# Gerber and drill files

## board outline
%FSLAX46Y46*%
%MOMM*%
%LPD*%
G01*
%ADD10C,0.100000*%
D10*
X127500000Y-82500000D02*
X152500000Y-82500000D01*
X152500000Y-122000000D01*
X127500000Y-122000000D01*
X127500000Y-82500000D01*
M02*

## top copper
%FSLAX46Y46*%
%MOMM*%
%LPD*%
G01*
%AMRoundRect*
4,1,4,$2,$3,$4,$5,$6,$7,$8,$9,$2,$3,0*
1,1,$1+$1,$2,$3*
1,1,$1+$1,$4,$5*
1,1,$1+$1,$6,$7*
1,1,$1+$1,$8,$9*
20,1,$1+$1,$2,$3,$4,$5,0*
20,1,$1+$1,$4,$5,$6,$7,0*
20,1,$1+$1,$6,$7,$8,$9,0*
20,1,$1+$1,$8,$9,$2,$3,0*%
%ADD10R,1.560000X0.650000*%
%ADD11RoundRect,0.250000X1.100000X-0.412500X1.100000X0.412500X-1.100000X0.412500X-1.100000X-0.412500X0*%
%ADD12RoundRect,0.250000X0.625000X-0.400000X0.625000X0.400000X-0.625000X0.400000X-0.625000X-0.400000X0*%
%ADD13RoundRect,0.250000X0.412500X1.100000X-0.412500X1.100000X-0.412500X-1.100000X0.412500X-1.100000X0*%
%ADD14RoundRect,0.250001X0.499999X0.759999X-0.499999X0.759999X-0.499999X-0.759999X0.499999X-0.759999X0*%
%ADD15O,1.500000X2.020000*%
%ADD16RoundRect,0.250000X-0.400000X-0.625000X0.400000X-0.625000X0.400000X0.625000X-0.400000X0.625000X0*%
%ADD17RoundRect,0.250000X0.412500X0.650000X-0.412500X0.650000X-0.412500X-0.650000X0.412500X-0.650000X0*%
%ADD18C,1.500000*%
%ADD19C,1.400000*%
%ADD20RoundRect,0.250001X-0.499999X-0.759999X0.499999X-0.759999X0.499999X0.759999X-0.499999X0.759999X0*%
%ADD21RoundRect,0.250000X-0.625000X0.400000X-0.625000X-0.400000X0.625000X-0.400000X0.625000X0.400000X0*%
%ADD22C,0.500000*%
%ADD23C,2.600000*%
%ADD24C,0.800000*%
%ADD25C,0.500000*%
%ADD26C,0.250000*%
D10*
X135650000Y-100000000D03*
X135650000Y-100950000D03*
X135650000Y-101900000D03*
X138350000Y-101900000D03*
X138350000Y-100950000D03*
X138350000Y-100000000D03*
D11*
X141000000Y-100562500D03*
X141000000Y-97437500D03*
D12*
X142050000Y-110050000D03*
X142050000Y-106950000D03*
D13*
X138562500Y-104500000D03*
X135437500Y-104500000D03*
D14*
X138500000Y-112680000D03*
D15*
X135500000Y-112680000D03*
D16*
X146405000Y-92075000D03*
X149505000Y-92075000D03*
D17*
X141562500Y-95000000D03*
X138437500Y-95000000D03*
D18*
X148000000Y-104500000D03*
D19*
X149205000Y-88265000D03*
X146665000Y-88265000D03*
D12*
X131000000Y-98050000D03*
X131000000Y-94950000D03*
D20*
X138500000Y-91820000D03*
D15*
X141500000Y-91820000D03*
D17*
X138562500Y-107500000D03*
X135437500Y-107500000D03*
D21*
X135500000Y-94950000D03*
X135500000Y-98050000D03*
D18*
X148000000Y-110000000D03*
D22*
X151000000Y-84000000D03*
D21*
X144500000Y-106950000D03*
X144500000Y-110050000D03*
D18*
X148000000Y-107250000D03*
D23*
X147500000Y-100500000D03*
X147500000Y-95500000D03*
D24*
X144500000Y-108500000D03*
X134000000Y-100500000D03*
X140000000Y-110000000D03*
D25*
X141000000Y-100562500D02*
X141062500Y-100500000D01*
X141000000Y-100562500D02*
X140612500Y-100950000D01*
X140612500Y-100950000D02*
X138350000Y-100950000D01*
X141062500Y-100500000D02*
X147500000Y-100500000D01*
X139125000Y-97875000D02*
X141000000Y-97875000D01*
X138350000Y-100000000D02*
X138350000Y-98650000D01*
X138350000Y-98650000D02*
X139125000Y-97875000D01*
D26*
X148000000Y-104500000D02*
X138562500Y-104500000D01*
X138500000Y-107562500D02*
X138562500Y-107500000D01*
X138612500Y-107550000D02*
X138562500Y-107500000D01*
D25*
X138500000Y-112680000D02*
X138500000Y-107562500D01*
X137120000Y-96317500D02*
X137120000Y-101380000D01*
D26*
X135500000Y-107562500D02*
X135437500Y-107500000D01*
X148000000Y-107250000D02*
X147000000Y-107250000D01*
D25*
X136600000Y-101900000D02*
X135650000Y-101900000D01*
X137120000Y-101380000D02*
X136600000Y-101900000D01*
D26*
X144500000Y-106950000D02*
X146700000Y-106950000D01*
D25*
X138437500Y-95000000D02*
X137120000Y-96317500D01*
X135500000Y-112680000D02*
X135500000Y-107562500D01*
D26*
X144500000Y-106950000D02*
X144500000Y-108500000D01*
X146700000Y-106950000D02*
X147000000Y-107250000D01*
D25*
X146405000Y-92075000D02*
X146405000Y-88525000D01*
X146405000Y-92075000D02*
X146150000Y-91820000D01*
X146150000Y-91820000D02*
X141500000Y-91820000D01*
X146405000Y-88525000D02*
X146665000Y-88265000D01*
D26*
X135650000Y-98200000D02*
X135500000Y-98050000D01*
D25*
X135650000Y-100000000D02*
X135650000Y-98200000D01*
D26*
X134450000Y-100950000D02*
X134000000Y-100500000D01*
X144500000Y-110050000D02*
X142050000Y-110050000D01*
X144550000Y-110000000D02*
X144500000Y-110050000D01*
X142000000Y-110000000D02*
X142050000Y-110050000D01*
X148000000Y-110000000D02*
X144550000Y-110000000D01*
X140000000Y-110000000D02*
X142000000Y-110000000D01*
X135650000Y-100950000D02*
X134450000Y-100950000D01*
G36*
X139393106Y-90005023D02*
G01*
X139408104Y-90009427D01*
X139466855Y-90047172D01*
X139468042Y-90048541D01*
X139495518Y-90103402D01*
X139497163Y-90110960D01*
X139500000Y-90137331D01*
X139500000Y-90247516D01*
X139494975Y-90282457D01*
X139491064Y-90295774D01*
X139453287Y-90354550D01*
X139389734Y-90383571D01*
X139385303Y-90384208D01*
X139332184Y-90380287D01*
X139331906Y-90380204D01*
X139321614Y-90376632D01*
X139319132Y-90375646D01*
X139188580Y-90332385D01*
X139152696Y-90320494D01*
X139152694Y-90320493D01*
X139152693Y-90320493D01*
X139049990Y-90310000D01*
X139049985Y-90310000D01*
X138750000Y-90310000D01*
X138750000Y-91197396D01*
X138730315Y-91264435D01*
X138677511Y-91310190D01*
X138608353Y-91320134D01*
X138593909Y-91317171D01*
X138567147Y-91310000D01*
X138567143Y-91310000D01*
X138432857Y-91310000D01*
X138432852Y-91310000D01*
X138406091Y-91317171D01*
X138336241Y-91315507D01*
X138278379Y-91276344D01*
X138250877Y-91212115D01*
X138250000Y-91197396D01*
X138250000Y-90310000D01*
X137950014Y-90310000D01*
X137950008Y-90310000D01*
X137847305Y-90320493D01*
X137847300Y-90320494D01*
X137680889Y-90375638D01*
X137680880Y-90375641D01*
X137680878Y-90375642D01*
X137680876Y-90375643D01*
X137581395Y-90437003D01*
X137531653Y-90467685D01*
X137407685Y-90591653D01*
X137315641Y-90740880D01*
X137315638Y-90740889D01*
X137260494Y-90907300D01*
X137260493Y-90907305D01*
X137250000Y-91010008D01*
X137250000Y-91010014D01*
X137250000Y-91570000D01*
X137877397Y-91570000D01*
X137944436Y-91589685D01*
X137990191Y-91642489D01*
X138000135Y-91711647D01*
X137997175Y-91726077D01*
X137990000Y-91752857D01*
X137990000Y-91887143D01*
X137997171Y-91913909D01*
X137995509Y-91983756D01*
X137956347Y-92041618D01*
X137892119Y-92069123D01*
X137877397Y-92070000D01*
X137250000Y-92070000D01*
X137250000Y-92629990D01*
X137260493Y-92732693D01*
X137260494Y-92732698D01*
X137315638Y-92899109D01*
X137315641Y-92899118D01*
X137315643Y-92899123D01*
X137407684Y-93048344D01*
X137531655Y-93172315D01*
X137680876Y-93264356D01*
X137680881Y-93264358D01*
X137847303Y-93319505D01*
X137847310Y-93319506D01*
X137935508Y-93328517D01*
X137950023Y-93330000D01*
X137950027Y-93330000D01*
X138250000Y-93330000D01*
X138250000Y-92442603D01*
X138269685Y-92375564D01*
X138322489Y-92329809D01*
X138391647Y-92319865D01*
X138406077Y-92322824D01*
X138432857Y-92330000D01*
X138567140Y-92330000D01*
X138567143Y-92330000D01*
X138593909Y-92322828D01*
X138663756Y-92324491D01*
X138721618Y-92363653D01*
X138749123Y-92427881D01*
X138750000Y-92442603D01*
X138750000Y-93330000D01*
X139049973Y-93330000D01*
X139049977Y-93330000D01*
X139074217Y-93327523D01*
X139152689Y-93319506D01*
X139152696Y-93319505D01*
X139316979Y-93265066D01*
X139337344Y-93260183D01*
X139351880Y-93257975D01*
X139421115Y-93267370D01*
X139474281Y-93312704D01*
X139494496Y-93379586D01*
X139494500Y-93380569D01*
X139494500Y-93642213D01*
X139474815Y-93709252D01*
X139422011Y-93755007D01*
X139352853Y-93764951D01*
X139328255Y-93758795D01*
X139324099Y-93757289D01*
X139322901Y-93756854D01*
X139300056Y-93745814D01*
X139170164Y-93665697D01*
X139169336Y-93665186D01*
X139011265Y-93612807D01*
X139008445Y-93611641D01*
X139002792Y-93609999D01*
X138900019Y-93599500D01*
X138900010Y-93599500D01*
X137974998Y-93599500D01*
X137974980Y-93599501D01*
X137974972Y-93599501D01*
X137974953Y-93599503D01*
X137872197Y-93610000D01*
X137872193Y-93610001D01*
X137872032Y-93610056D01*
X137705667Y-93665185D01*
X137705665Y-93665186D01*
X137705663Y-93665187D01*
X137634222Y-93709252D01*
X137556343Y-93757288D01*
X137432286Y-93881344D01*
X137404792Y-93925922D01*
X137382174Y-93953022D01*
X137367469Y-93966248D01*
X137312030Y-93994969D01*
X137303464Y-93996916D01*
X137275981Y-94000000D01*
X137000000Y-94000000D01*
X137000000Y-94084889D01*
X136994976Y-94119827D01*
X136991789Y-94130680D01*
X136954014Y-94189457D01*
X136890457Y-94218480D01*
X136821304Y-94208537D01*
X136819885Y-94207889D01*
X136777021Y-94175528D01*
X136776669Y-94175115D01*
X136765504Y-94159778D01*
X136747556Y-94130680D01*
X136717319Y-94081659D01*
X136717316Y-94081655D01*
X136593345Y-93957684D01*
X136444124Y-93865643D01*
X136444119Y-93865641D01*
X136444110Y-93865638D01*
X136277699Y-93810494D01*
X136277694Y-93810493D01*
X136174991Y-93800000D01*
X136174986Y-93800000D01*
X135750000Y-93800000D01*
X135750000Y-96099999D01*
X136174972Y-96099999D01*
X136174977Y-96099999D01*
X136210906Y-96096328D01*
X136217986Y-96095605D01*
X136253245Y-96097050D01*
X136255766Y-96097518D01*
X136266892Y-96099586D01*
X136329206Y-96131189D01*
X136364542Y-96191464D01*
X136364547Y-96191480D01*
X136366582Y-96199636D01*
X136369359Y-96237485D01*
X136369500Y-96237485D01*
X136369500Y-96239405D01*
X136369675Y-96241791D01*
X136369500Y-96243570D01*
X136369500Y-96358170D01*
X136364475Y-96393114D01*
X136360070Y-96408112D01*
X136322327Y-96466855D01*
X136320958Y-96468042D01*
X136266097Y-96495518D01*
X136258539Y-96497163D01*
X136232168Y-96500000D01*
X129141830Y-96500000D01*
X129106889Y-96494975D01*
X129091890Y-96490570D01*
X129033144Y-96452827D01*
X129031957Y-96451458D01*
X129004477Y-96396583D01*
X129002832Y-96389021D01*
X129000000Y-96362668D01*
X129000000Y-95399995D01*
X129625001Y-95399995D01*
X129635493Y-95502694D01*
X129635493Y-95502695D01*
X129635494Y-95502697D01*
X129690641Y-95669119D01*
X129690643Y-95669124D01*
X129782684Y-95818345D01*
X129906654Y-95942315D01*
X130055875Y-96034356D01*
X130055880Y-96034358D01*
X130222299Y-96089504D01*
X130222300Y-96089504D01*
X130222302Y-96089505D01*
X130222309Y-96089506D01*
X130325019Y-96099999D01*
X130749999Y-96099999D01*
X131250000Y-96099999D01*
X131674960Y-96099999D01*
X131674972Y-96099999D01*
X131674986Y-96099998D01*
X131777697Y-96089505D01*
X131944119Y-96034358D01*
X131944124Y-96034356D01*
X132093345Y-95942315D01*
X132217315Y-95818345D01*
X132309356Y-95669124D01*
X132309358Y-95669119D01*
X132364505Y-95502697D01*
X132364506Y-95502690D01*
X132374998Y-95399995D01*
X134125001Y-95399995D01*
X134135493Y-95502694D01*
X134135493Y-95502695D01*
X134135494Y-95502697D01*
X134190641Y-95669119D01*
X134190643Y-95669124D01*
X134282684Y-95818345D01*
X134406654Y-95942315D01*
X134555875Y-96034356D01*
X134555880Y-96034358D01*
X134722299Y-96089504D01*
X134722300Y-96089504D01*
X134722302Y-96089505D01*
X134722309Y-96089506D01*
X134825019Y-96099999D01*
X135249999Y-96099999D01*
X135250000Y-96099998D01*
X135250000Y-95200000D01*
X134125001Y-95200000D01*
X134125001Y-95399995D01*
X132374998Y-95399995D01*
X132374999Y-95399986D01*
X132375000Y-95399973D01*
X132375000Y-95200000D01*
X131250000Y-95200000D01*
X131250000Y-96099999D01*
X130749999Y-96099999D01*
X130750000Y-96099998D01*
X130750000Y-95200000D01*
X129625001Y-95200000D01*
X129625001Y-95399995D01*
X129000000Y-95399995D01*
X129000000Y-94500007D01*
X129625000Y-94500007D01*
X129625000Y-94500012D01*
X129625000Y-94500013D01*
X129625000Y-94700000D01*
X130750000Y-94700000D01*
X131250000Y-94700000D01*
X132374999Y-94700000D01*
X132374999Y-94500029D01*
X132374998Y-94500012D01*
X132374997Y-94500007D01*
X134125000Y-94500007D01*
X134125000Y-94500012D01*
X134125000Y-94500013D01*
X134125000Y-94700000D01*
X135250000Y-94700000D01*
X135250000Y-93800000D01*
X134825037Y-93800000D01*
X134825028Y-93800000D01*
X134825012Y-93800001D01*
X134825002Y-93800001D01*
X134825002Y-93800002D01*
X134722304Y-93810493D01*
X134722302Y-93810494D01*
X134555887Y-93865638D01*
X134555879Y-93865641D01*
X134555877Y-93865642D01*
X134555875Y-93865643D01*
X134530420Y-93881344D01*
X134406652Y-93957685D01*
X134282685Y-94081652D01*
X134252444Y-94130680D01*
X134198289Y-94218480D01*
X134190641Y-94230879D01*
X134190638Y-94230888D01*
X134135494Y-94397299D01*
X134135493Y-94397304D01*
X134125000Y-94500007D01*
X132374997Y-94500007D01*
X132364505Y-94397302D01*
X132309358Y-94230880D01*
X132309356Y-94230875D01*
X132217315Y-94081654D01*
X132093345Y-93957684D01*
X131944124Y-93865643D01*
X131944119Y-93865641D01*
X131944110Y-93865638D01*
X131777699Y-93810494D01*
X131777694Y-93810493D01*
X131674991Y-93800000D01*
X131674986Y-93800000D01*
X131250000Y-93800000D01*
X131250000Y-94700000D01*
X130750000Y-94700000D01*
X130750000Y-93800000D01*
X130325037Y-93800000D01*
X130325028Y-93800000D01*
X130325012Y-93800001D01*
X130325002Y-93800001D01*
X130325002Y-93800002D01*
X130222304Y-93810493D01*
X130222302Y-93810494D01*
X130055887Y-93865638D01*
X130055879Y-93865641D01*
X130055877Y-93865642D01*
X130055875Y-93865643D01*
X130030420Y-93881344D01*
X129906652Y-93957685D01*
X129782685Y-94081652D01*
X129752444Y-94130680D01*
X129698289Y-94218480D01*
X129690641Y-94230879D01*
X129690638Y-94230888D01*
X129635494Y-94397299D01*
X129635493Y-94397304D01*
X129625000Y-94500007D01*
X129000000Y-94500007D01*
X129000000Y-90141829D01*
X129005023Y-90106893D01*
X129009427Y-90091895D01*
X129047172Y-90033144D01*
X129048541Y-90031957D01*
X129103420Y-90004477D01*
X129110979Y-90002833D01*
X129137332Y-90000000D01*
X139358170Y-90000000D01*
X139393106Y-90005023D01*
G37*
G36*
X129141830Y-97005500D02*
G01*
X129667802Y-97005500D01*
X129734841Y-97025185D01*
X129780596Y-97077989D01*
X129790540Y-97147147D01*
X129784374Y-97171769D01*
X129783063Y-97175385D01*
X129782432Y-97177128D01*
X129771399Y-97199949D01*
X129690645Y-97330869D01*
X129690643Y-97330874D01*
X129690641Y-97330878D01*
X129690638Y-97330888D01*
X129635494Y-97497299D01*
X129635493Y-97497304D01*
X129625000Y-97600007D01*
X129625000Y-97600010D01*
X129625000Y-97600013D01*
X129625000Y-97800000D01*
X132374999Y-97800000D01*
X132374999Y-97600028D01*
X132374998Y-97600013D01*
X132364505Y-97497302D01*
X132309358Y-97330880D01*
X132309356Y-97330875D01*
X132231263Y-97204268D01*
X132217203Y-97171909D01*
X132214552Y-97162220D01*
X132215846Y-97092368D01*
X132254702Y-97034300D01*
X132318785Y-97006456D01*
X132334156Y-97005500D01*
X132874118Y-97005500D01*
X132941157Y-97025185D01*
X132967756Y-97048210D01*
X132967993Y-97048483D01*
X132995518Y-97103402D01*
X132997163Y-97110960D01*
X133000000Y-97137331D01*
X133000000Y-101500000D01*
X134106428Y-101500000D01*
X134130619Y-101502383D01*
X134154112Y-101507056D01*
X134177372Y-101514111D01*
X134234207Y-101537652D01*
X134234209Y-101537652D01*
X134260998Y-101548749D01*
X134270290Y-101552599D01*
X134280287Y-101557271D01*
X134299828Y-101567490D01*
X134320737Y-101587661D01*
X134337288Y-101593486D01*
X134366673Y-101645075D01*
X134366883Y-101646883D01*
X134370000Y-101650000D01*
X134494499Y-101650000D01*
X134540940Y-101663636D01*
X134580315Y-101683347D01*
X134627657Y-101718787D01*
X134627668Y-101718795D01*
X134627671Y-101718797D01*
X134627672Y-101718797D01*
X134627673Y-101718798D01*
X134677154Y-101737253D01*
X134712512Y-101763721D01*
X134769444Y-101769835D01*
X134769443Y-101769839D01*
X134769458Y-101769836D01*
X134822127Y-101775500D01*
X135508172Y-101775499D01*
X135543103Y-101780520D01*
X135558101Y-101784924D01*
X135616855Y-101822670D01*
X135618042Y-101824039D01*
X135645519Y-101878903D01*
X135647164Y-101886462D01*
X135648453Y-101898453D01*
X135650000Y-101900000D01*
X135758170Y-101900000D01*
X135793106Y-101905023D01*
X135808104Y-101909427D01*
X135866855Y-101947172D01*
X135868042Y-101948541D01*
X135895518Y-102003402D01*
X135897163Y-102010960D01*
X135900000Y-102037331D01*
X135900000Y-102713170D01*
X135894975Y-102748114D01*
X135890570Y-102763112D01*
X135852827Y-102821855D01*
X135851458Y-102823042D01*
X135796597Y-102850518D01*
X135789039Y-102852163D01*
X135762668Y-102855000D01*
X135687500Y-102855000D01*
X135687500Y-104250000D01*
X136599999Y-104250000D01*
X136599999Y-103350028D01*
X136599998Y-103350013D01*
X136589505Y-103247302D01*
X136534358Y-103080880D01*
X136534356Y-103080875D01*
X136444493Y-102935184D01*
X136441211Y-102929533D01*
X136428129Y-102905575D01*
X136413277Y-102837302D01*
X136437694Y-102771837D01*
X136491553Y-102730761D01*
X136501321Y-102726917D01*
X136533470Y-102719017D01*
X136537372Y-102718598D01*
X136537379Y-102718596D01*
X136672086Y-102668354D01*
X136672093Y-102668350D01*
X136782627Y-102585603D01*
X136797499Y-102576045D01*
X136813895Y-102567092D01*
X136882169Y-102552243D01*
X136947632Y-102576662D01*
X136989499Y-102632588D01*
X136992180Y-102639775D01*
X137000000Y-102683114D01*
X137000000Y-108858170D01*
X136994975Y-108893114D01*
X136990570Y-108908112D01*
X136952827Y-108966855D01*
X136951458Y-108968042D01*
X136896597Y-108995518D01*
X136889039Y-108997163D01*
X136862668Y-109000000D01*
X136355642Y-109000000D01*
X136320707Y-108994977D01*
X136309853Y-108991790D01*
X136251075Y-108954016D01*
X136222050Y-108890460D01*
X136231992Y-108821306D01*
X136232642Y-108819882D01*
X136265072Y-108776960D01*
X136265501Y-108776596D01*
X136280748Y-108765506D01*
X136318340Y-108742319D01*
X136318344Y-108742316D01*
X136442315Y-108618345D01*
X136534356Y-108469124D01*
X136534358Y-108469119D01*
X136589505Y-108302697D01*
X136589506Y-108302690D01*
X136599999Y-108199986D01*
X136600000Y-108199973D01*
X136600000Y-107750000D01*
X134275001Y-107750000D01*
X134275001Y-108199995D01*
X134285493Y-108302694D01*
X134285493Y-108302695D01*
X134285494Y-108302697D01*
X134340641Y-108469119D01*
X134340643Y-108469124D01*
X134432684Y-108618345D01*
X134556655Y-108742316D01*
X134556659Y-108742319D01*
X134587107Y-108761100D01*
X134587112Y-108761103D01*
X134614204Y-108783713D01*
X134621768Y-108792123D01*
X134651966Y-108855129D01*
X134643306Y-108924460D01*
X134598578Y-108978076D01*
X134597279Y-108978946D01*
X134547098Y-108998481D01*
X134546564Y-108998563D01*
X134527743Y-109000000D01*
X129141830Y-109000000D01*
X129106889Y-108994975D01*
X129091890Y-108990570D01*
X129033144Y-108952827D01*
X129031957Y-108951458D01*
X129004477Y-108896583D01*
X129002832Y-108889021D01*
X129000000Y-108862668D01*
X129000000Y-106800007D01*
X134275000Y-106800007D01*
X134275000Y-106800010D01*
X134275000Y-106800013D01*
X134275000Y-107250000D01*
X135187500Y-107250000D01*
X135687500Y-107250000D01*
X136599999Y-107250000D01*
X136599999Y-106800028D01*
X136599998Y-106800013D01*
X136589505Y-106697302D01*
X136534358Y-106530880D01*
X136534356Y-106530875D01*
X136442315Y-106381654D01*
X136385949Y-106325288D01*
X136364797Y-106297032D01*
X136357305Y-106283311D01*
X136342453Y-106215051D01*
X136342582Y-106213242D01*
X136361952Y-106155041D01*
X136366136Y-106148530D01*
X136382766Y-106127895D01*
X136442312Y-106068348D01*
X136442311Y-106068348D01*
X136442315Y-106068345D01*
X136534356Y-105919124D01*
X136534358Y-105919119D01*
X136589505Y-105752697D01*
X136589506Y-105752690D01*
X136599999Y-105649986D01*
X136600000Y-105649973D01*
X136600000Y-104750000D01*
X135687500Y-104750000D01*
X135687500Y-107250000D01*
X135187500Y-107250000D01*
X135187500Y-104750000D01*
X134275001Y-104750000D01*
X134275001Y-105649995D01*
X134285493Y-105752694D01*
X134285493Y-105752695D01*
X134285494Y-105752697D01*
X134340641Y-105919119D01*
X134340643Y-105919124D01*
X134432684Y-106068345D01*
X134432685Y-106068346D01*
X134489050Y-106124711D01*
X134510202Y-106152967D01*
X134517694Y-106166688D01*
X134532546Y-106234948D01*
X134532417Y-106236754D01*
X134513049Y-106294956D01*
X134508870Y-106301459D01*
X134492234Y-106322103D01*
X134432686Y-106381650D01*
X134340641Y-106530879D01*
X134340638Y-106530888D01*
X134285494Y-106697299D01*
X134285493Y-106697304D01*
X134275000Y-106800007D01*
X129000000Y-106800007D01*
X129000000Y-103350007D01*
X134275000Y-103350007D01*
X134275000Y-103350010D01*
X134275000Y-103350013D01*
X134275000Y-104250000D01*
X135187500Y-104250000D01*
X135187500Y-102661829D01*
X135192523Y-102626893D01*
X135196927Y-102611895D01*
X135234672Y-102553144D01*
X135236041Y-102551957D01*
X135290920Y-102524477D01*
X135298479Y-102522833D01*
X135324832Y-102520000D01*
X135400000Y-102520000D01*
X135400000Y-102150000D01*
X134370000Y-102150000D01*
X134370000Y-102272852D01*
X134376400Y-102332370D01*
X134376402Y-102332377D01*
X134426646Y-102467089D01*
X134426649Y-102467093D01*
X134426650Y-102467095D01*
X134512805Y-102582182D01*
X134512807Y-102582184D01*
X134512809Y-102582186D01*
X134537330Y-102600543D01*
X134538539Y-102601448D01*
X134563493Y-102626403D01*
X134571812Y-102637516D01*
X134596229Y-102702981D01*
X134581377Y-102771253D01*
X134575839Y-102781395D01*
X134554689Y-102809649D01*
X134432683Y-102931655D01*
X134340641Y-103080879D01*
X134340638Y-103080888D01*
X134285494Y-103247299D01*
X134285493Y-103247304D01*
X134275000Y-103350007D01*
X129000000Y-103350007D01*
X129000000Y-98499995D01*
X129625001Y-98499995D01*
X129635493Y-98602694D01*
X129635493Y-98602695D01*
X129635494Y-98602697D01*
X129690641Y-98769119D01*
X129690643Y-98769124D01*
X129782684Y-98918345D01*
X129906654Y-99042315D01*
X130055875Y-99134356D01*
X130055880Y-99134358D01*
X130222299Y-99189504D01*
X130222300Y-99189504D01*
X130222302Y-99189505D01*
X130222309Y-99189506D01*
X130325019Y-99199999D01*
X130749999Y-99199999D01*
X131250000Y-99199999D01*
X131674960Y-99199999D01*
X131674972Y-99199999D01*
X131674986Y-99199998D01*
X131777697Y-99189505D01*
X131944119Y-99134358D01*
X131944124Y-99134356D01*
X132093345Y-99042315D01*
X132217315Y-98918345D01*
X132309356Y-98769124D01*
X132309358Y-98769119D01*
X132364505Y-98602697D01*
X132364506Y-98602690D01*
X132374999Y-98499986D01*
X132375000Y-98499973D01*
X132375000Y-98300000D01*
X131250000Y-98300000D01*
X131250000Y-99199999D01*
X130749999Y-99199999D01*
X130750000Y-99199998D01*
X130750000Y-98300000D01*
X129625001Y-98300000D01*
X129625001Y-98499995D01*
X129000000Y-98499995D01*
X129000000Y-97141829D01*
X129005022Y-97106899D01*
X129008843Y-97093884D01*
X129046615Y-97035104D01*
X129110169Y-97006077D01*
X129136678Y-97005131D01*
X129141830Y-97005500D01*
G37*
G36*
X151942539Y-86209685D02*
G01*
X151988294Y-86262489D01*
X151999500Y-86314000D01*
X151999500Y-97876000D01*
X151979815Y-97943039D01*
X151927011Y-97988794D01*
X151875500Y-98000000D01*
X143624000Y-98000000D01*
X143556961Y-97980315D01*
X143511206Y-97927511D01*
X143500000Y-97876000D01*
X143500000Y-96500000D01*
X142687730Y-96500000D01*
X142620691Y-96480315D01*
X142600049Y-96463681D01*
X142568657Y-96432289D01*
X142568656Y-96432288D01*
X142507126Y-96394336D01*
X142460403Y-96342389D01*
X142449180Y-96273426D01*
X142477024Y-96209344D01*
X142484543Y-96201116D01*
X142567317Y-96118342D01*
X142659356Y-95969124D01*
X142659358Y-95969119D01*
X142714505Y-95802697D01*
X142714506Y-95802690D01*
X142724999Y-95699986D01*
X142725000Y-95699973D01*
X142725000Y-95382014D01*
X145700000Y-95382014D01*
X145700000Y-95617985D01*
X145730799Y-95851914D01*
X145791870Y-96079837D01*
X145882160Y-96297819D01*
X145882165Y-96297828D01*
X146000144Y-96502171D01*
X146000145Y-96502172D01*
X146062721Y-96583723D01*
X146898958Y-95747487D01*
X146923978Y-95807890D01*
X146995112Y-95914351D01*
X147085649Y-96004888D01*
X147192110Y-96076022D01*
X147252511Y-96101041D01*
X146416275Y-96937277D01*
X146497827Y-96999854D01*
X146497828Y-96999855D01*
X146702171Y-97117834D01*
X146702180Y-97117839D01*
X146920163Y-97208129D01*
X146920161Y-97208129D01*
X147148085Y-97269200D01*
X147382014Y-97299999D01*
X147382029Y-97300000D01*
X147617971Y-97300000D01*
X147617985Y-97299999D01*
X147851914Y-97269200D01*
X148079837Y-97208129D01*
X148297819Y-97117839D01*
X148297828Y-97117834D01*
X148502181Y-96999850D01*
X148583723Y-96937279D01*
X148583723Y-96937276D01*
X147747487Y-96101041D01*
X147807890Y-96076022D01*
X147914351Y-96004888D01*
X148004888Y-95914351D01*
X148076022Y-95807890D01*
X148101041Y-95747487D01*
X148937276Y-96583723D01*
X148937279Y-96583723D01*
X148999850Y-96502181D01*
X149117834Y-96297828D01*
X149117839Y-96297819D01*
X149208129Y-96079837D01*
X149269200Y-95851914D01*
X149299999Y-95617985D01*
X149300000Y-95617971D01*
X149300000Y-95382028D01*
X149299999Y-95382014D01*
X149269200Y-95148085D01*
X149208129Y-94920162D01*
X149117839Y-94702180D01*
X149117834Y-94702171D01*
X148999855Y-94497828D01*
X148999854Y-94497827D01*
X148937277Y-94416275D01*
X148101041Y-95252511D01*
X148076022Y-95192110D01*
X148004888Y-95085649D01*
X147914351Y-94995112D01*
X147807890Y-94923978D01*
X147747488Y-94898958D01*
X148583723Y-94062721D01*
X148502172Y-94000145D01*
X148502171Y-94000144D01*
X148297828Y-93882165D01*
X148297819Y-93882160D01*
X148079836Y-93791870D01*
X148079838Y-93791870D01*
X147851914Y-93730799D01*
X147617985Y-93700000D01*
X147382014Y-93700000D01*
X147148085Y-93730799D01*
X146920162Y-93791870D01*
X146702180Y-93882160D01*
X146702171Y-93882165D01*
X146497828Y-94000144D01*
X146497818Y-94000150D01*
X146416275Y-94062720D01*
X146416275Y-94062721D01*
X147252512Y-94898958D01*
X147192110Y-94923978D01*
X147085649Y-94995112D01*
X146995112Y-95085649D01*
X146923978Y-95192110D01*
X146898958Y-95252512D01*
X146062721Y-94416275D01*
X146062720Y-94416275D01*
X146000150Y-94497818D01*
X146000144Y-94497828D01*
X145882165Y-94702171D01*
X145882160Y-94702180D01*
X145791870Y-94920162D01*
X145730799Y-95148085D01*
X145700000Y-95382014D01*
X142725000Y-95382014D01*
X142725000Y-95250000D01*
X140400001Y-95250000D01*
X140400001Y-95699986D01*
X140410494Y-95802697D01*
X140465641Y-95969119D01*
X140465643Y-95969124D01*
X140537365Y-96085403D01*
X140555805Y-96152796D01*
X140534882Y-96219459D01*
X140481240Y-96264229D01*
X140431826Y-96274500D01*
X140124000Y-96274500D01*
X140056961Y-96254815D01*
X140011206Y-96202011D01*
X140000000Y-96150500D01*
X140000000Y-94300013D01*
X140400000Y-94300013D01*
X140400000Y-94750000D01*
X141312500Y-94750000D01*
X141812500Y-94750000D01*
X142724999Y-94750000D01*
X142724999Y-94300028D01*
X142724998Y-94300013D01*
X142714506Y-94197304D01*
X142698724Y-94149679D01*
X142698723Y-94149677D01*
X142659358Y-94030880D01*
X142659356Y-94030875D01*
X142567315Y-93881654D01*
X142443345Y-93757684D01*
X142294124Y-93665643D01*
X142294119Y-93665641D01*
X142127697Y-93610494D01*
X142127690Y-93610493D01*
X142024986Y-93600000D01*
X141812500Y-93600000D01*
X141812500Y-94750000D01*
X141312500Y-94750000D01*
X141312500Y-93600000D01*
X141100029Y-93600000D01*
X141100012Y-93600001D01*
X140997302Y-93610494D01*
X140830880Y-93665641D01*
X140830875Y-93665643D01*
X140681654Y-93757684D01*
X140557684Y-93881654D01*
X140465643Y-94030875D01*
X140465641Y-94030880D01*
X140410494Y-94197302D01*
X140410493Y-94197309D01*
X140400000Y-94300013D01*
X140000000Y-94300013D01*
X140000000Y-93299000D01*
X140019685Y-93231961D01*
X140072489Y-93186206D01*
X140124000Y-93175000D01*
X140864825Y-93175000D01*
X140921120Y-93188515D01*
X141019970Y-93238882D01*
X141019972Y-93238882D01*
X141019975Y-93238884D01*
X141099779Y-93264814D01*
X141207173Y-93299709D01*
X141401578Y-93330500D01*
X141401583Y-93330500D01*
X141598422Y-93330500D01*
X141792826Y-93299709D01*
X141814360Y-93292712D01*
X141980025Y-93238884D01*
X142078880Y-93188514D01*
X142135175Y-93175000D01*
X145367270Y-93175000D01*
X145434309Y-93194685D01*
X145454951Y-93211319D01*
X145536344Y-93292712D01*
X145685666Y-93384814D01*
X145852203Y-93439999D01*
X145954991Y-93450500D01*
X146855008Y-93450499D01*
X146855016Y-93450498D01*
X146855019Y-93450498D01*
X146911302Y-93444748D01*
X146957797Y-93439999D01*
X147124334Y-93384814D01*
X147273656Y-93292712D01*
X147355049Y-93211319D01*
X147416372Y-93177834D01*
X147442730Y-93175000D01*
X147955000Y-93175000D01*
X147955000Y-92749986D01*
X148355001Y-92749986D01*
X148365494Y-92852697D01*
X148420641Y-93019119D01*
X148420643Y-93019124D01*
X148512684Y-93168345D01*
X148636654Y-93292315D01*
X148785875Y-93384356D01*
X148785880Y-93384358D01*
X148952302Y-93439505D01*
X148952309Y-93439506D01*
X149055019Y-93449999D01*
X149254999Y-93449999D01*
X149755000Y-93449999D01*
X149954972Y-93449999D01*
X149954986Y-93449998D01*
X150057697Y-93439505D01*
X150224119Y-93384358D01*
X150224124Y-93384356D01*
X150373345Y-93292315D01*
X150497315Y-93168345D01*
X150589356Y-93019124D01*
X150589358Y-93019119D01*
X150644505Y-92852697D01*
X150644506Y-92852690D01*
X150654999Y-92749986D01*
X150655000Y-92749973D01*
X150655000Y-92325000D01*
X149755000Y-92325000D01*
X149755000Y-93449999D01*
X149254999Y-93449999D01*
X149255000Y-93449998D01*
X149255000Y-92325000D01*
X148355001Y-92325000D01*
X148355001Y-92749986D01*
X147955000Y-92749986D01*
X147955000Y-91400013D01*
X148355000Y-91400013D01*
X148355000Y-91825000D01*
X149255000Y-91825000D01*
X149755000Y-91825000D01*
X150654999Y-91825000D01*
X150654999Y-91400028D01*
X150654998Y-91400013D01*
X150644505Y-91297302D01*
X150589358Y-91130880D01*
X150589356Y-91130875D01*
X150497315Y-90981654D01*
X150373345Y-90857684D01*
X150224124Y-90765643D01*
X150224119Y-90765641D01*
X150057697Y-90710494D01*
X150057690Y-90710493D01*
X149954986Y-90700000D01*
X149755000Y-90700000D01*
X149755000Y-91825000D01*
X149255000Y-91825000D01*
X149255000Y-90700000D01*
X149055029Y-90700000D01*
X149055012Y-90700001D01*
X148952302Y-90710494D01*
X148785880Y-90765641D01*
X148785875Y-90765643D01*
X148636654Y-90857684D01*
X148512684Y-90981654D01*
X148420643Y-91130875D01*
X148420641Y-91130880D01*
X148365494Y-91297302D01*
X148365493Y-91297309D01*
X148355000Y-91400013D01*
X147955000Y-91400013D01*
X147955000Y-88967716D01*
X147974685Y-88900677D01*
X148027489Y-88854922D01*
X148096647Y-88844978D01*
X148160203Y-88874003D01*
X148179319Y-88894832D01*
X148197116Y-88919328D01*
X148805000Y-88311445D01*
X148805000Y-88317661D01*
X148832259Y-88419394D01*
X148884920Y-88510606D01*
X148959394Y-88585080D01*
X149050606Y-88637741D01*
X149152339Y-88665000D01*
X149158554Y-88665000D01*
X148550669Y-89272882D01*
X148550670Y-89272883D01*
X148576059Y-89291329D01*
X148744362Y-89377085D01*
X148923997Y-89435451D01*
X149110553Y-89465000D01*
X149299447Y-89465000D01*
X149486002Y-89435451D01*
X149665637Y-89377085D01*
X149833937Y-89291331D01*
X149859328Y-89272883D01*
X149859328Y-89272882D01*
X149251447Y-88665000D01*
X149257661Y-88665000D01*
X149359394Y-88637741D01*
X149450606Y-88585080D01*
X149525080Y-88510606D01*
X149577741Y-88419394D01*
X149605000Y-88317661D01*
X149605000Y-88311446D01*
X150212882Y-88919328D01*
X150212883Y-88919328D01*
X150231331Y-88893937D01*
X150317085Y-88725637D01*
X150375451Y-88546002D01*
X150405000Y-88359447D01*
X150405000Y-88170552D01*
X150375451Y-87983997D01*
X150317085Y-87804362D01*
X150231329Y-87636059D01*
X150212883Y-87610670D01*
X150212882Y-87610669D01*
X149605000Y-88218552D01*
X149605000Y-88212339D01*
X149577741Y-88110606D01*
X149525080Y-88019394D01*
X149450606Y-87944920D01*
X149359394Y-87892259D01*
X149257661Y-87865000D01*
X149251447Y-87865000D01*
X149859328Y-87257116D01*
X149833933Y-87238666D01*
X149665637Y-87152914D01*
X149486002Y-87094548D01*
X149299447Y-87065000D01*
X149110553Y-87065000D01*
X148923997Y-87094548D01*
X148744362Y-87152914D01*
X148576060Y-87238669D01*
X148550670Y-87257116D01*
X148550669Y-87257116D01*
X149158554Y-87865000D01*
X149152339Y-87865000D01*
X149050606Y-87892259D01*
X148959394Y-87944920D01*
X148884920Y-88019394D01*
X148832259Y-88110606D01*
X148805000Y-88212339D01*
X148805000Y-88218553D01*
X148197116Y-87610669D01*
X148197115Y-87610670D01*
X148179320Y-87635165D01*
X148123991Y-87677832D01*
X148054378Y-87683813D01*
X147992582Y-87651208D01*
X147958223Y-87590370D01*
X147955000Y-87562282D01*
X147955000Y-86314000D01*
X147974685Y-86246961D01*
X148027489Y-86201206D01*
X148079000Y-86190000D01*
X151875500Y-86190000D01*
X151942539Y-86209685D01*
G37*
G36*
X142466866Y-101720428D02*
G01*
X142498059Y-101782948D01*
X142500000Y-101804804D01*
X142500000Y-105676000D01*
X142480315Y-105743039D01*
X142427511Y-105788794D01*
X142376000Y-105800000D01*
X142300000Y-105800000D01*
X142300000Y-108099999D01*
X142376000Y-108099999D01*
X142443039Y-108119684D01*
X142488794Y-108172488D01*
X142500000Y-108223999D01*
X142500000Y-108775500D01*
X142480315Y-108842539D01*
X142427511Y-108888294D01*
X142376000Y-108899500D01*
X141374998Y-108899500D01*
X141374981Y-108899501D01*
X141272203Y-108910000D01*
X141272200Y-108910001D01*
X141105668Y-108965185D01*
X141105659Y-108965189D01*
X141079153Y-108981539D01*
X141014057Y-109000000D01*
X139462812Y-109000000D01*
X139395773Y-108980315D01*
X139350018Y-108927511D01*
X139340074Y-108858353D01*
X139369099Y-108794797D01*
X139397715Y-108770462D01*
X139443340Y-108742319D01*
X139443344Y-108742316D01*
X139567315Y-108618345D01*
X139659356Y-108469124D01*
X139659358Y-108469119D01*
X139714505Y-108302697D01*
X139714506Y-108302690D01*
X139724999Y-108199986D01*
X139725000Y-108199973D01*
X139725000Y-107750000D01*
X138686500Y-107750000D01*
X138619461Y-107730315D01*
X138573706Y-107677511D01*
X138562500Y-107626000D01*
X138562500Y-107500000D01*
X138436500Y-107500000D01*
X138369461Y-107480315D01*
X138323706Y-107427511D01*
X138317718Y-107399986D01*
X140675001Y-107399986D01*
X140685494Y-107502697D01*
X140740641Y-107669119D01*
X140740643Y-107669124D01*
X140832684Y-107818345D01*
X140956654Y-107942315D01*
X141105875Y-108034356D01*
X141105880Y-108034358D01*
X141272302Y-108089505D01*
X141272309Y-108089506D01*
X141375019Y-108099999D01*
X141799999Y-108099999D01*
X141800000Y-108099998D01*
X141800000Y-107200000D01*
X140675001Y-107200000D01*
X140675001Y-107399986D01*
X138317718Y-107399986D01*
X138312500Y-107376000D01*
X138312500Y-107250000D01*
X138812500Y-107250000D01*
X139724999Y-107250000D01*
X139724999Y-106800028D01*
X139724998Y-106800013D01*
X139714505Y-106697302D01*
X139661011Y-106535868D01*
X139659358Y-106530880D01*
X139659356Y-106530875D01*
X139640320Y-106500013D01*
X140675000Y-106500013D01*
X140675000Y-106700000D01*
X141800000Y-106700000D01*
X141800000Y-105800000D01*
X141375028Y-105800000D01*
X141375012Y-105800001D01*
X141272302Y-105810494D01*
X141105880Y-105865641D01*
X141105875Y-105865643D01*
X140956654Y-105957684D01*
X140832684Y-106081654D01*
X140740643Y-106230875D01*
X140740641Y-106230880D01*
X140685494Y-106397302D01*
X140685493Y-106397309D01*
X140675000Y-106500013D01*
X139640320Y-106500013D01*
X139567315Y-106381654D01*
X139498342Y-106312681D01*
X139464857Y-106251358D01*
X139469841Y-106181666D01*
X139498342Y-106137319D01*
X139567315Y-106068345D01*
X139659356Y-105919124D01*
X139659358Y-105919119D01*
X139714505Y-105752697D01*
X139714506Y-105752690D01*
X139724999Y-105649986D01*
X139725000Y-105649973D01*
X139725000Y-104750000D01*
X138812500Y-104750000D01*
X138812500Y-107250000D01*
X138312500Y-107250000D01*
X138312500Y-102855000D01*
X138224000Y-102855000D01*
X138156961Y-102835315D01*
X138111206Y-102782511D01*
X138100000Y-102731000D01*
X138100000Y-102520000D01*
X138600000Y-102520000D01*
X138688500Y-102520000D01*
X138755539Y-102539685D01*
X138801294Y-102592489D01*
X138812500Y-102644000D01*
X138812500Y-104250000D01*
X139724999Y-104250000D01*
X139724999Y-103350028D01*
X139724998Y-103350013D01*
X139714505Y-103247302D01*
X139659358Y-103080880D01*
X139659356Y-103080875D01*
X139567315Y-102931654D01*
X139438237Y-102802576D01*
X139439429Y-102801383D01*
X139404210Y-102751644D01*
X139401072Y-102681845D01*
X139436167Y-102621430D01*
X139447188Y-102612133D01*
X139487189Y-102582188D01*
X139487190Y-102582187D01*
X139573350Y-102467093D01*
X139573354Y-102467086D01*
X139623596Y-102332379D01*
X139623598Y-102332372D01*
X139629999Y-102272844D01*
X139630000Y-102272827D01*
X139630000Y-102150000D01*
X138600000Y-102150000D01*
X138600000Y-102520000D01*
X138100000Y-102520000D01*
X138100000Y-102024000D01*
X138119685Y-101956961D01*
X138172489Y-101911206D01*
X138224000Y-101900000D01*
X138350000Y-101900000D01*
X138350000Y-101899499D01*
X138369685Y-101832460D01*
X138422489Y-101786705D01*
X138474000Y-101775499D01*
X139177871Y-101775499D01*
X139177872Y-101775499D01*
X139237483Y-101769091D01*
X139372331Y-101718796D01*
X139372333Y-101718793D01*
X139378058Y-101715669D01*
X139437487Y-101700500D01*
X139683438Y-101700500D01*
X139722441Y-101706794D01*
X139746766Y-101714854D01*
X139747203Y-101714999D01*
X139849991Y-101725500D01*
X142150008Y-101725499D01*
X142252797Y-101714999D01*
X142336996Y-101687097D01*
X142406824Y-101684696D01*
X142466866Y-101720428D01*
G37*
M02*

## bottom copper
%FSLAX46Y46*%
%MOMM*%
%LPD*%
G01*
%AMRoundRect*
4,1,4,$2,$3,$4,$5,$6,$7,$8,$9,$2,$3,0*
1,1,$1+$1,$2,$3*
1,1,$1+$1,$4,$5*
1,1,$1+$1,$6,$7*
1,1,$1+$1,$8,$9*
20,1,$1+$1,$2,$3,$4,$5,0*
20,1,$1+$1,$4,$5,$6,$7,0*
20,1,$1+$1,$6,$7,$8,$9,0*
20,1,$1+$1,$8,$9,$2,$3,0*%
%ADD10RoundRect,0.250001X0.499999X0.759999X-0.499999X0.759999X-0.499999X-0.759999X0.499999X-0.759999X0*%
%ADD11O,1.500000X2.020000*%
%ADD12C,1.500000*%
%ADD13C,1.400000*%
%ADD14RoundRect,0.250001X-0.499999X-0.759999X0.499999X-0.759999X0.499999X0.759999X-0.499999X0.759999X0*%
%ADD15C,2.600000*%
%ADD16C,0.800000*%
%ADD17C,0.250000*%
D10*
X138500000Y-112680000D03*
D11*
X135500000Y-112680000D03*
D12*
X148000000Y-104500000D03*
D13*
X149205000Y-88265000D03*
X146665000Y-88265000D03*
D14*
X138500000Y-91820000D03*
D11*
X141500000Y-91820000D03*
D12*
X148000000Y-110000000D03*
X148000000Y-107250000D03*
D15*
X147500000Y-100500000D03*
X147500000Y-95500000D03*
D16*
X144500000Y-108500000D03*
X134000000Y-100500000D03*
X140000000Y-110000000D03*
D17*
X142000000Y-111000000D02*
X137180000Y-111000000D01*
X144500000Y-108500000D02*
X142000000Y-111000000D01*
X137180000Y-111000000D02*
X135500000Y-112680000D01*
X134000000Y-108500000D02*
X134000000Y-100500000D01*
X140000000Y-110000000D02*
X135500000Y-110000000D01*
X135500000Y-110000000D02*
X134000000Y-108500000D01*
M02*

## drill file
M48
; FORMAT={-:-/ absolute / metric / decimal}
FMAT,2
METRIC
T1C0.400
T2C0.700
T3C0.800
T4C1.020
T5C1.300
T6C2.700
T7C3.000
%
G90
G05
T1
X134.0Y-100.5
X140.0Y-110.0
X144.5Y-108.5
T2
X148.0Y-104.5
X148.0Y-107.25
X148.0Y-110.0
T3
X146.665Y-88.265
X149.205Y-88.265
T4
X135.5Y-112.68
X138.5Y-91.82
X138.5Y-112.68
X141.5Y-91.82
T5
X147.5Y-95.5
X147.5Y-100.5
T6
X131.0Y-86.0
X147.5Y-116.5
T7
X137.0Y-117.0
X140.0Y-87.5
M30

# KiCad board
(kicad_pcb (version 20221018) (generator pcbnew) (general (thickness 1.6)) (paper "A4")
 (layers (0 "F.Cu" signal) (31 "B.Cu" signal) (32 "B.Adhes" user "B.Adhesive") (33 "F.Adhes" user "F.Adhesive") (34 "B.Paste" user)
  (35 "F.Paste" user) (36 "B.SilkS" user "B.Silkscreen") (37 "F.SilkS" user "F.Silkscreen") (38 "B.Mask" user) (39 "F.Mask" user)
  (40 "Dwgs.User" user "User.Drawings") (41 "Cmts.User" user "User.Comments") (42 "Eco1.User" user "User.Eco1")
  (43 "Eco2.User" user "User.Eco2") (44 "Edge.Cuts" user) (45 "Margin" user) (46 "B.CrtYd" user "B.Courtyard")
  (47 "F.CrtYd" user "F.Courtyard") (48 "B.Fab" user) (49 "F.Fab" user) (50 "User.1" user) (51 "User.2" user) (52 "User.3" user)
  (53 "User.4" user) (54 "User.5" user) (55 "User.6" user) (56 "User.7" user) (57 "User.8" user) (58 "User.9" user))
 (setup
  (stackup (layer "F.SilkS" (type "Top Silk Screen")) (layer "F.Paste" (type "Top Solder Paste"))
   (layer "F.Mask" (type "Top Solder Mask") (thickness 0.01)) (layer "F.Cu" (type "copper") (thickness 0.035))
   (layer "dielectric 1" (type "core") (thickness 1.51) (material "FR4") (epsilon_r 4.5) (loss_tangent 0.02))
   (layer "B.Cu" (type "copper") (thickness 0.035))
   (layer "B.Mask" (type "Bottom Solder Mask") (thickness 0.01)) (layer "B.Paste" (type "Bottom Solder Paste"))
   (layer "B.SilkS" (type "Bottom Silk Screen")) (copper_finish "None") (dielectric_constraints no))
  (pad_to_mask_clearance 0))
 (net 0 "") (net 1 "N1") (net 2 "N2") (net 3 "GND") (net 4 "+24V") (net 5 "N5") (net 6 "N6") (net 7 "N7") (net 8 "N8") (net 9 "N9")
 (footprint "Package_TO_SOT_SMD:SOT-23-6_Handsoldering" (layer "F.Cu") (at 137 100.95)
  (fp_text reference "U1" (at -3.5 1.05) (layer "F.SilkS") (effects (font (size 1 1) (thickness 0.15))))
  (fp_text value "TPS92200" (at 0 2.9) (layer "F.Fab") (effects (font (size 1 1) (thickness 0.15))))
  (pad "1" smd rect (at -1.35 -0.95) (size 1.56 0.65) (layers "F.Cu" "F.Paste" "F.Mask") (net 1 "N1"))
  (pad "2" smd rect (at -1.35 0) (size 1.56 0.65) (layers "F.Cu" "F.Paste" "F.Mask") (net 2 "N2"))
  (pad "3" smd rect (at -1.35 0.95) (size 1.56 0.65) (layers "F.Cu" "F.Paste" "F.Mask") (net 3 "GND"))
  (pad "4" smd rect (at 1.35 0.95) (size 1.56 0.65) (layers "F.Cu" "F.Paste" "F.Mask") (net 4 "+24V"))
  (pad "5" smd rect (at 1.35 0) (size 1.56 0.65) (layers "F.Cu" "F.Paste" "F.Mask") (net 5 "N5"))
  (pad "6" smd rect (at 1.35 -0.95) (size 1.56 0.65) (layers "F.Cu" "F.Paste" "F.Mask") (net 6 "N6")))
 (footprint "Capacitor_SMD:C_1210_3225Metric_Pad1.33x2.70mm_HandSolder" (layer "F.Cu") (at 141 99 90)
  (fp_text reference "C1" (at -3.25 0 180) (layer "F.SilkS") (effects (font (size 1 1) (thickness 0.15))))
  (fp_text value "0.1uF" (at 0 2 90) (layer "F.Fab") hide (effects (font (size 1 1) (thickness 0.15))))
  (pad "1" smd roundrect (at -1.5625 0 90) (size 1.325 2.7) (layers "F.Cu" "F.Paste" "F.Mask") (roundrect_rratio 0.188679) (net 5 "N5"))
  (pad "2" smd roundrect (at 1.5625 0 90) (size 1.325 2.7) (layers "F.Cu" "F.Paste" "F.Mask") (roundrect_rratio 0.188679) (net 6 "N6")))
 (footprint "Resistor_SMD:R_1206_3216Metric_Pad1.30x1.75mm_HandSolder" (layer "F.Cu") (at 142.05 108.5 90)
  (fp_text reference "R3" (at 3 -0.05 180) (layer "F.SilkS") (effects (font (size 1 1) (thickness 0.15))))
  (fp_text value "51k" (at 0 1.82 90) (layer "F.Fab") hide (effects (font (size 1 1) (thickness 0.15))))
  (pad "1" smd roundrect (at -1.55 0 90) (size 1.3 1.75) (layers "F.Cu" "F.Paste" "F.Mask") (roundrect_rratio 0.192308) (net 2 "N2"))
  (pad "2" smd roundrect (at 1.55 0 90) (size 1.3 1.75) (layers "F.Cu" "F.Paste" "F.Mask") (roundrect_rratio 0.192308) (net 4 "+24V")))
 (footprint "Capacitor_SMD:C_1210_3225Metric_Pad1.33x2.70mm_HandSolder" (layer "F.Cu") (at 137 104.5 180)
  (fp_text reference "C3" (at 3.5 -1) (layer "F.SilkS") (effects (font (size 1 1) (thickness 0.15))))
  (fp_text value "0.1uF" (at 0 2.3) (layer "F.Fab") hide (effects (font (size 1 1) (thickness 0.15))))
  (pad "1" smd roundrect (at -1.5625 0 180) (size 1.325 2.7) (layers "F.Cu" "F.Paste" "F.Mask") (roundrect_rratio 0.188679) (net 4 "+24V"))
  (pad "2" smd roundrect (at 1.5625 0 180) (size 1.325 2.7) (layers "F.Cu" "F.Paste" "F.Mask") (roundrect_rratio 0.188679) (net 3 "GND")))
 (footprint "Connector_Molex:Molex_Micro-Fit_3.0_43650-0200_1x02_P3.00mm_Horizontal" (layer "F.Cu") (at 138.5 112.68 180)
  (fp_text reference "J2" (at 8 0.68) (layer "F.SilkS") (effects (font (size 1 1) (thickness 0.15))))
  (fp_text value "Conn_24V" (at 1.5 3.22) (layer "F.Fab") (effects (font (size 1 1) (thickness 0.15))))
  (pad "" np_thru_hole circle (at 1.5 -4.32 180) (size 3 3) (drill 3) (layers "*.Cu" "*.Mask"))
  (pad "1" thru_hole roundrect (at 0 0 180) (size 1.5 2.02) (drill 1.02) (layers "*.Cu" "*.Mask") (roundrect_rratio 0.166667) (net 4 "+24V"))
  (pad "2" thru_hole oval (at 3 0 180) (size 1.5 2.02) (drill 1.02) (layers "*.Cu" "*.Mask") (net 3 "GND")))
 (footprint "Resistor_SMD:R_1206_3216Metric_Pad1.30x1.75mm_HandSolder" (layer "F.Cu") (at 147.955 92.075)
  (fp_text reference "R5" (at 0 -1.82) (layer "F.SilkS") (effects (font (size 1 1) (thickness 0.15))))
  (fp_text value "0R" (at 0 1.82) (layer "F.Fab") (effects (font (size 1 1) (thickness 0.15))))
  (pad "1" smd roundrect (at -1.55 0) (size 1.3 1.75) (layers "F.Cu" "F.Paste" "F.Mask") (roundrect_rratio 0.192308) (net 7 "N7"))
  (pad "2" smd roundrect (at 1.55 0) (size 1.3 1.75) (layers "F.Cu" "F.Paste" "F.Mask") (roundrect_rratio 0.192308) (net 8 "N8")))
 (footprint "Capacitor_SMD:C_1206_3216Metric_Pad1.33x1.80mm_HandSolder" (layer "F.Cu") (at 140 95 180)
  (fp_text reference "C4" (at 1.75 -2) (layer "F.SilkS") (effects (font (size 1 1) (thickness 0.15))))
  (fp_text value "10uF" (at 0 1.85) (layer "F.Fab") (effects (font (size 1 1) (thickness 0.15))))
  (pad "1" smd roundrect (at -1.5625 0 180) (size 1.325 1.8) (layers "F.Cu" "F.Paste" "F.Mask") (roundrect_rratio 0.188679) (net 8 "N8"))
  (pad "2" smd roundrect (at 1.5625 0 180) (size 1.325 1.8) (layers "F.Cu" "F.Paste" "F.Mask") (roundrect_rratio 0.188679) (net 3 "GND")))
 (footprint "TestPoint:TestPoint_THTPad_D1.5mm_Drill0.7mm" (layer "F.Cu") (at 148 104.5)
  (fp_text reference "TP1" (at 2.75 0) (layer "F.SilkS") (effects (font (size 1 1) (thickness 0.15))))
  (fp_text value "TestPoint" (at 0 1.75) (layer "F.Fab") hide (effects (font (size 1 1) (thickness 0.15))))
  (pad "1" thru_hole circle (at 0 0) (size 1.5 1.5) (drill 0.7) (layers "*.Cu" "*.Mask") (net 4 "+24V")))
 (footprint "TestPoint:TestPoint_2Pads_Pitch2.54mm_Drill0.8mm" (layer "F.Cu") (at 149.205 88.265 180)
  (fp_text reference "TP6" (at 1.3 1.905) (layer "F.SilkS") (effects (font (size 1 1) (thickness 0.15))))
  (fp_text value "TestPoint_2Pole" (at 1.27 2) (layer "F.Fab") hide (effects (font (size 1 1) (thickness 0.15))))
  (pad "1" thru_hole circle (at 0 0 180) (size 1.4 1.4) (drill 0.8) (layers "*.Cu" "*.Mask") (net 8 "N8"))
  (pad "2" thru_hole circle (at 2.54 0 180) (size 1.4 1.4) (drill 0.8) (layers "*.Cu" "*.Mask") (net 7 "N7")))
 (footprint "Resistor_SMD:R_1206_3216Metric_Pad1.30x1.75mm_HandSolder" (layer "F.Cu") (at 131 96.5 90)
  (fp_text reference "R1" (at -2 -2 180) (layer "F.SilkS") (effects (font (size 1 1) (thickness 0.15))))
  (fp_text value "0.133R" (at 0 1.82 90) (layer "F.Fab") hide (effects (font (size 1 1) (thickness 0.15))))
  (pad "1" smd roundrect (at -1.55 0 90) (size 1.3 1.75) (layers "F.Cu" "F.Paste" "F.Mask") (roundrect_rratio 0.192308) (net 3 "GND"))
  (pad "2" smd roundrect (at 1.55 0 90) (size 1.3 1.75) (layers "F.Cu" "F.Paste" "F.Mask") (roundrect_rratio 0.192308) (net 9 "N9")))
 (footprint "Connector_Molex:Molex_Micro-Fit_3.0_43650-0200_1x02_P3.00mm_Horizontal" (layer "F.Cu") (at 138.5 91.82)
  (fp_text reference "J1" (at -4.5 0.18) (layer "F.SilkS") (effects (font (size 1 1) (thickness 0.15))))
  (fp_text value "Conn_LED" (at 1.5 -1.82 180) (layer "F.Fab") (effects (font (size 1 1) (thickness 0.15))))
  (pad "" np_thru_hole circle (at 1.5 -4.32) (size 3 3) (drill 3) (layers "*.Cu" "*.Mask"))
  (pad "1" thru_hole roundrect (at 0 0) (size 1.5 2.02) (drill 1.02) (layers "*.Cu" "*.Mask") (roundrect_rratio 0.166667) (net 9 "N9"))
  (pad "2" thru_hole oval (at 3 0) (size 1.5 2.02) (drill 1.02) (layers "*.Cu" "*.Mask") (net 7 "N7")))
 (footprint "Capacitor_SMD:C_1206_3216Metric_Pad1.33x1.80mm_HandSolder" (layer "F.Cu") (at 137 107.5 180)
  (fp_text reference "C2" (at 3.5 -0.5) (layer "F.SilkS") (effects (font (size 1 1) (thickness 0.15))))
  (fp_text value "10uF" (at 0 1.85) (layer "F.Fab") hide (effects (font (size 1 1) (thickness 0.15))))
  (pad "1" smd roundrect (at -1.5625 0 180) (size 1.325 1.8) (layers "F.Cu" "F.Paste" "F.Mask") (roundrect_rratio 0.188679) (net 4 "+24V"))
  (pad "2" smd roundrect (at 1.5625 0 180) (size 1.325 1.8) (layers "F.Cu" "F.Paste" "F.Mask") (roundrect_rratio 0.188679) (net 3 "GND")))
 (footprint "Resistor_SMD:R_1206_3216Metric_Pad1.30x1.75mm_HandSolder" (layer "F.Cu") (at 135.5 96.5 -90)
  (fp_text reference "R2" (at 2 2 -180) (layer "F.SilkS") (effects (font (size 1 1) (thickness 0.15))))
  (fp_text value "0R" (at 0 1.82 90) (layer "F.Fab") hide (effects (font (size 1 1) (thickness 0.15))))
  (pad "1" smd roundrect (at -1.55 0 270) (size 1.3 1.75) (layers "F.Cu" "F.Paste" "F.Mask") (roundrect_rratio 0.192308) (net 9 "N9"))
  (pad "2" smd roundrect (at 1.55 0 270) (size 1.3 1.75) (layers "F.Cu" "F.Paste" "F.Mask") (roundrect_rratio 0.192308) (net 1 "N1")))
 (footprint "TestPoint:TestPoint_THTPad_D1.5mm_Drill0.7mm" (layer "F.Cu") (at 148 110)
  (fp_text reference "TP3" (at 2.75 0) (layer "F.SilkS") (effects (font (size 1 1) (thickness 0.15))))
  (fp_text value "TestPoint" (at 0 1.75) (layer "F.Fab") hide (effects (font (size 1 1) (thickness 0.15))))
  (pad "1" thru_hole circle (at 0 0) (size 1.5 1.5) (drill 0.7) (layers "*.Cu" "*.Mask") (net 2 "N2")))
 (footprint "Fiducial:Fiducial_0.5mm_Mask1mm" (layer "F.Cu") (at 151 84)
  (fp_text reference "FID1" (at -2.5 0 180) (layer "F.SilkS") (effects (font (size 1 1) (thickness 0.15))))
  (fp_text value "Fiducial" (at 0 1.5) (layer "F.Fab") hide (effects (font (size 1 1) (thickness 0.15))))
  (pad "" smd circle (at 0 0) (size 0.5 0.5) (layers "F.Cu" "F.Mask") (solder_mask_margin 0.25) (clearance 0.25)))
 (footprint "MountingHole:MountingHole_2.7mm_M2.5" (layer "F.Cu") (at 147.5 116.5)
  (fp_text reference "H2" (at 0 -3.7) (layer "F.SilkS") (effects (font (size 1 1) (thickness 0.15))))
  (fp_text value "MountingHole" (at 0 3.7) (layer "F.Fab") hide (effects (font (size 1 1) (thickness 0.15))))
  (pad "" np_thru_hole circle (at 0 0) (size 2.7 2.7) (drill 2.7) (layers "*.Cu" "*.Mask")))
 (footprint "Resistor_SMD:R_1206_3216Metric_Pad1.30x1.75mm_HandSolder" (layer "F.Cu") (at 144.5 108.5 -90)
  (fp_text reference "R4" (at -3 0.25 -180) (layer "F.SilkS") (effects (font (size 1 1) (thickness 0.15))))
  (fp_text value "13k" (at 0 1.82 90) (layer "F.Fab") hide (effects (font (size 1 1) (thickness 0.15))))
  (pad "1" smd roundrect (at -1.55 0 270) (size 1.3 1.75) (layers "F.Cu" "F.Paste" "F.Mask") (roundrect_rratio 0.192308) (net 3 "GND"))
  (pad "2" smd roundrect (at 1.55 0 270) (size 1.3 1.75) (layers "F.Cu" "F.Paste" "F.Mask") (roundrect_rratio 0.192308) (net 2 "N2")))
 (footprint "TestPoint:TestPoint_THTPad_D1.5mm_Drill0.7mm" (layer "F.Cu") (at 148 107.25)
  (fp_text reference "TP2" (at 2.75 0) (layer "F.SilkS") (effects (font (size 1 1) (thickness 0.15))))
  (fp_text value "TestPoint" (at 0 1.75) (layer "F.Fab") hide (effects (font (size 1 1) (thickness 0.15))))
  (pad "1" thru_hole circle (at 0 0) (size 1.5 1.5) (drill 0.7) (layers "*.Cu" "*.Mask") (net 3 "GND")))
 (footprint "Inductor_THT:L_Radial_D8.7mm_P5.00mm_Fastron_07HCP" (layer "F.Cu") (at 147.5 100.5 90)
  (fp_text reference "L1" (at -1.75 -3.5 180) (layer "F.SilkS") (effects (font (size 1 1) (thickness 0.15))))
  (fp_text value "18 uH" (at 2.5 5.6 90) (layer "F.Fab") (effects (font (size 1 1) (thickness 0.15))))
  (pad "1" thru_hole circle (at 0 0 90) (size 2.6 2.6) (drill 1.3) (layers "*.Cu" "*.Mask") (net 5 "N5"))
  (pad "2" thru_hole circle (at 5 0 90) (size 2.6 2.6) (drill 1.3) (layers "*.Cu" "*.Mask") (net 8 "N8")))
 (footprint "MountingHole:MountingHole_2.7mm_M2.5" (layer "F.Cu") (at 131 86)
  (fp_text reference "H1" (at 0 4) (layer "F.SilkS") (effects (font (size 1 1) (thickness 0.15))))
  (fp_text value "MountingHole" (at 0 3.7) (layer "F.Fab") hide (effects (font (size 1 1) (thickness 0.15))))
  (pad "" np_thru_hole circle (at 0 0) (size 2.7 2.7) (drill 2.7) (layers "*.Cu" "*.Mask")))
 (gr_rect (start 127.5 82.5) (end 152.5 122) (stroke (width 0.1) (type default)) (fill none) (layer "Edge.Cuts"))
 (segment (start 141 100.5625) (end 141.0625 100.5) (width 0.5) (layer "F.Cu") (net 5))
 (segment (start 141 100.5625) (end 140.6125 100.95) (width 0.5) (layer "F.Cu") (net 5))
 (segment (start 140.6125 100.95) (end 138.35 100.95) (width 0.5) (layer "F.Cu") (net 5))
 (segment (start 141.0625 100.5) (end 147.5 100.5) (width 0.5) (layer "F.Cu") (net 5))
 (segment (start 139.125 97.875) (end 141 97.875) (width 0.5) (layer "F.Cu") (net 6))
 (segment (start 138.35 100) (end 138.35 98.65) (width 0.5) (layer "F.Cu") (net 6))
 (segment (start 138.35 98.65) (end 139.125 97.875) (width 0.5) (layer "F.Cu") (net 6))
 (segment (start 148 104.5) (end 138.5625 104.5) (width 0.25) (layer "F.Cu") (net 4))
 (segment (start 138.5 107.5625) (end 138.5625 107.5) (width 0.25) (layer "F.Cu") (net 4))
 (segment (start 138.6125 107.55) (end 138.5625 107.5) (width 0.25) (layer "F.Cu") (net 4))
 (segment (start 138.5 112.68) (end 138.5 107.5625) (width 0.5) (layer "F.Cu") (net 4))
 (segment (start 137.12 96.3175) (end 137.12 101.38) (width 0.5) (layer "F.Cu") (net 3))
 (segment (start 135.5 107.5625) (end 135.4375 107.5) (width 0.25) (layer "F.Cu") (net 3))
 (segment (start 148 107.25) (end 147 107.25) (width 0.25) (layer "F.Cu") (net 3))
 (segment (start 136.6 101.9) (end 135.65 101.9) (width 0.5) (layer "F.Cu") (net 3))
 (segment (start 137.12 101.38) (end 136.6 101.9) (width 0.5) (layer "F.Cu") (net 3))
 (segment (start 144.5 106.95) (end 146.7 106.95) (width 0.25) (layer "F.Cu") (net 3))
 (segment (start 138.4375 95) (end 137.12 96.3175) (width 0.5) (layer "F.Cu") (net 3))
 (segment (start 135.5 112.68) (end 135.5 107.5625) (width 0.5) (layer "F.Cu") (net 3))
 (segment (start 144.5 106.95) (end 144.5 108.5) (width 0.25) (layer "F.Cu") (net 3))
 (segment (start 146.7 106.95) (end 147 107.25) (width 0.25) (layer "F.Cu") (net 3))
 (via (at 144.5 108.5) (size 0.8) (drill 0.4) (layers "F.Cu" "B.Cu") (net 3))
 (segment (start 142 111) (end 137.18 111) (width 0.25) (layer "B.Cu") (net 3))
 (segment (start 144.5 108.5) (end 142 111) (width 0.25) (layer "B.Cu") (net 3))
 (segment (start 137.18 111) (end 135.5 112.68) (width 0.25) (layer "B.Cu") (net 3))
 (segment (start 146.405 92.075) (end 146.405 88.525) (width 0.5) (layer "F.Cu") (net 7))
 (segment (start 146.405 92.075) (end 146.15 91.82) (width 0.5) (layer "F.Cu") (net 7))
 (segment (start 146.15 91.82) (end 141.5 91.82) (width 0.5) (layer "F.Cu") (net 7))
 (segment (start 146.405 88.525) (end 146.665 88.265) (width 0.5) (layer "F.Cu") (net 7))
 (segment (start 135.65 98.2) (end 135.5 98.05) (width 0.25) (layer "F.Cu") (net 1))
 (segment (start 135.65 100) (end 135.65 98.2) (width 0.5) (layer "F.Cu") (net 1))
 (segment (start 134.45 100.95) (end 134 100.5) (width 0.25) (layer "F.Cu") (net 2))
 (segment (start 144.5 110.05) (end 142.05 110.05) (width 0.25) (layer "F.Cu") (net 2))
 (segment (start 144.55 110) (end 144.5 110.05) (width 0.25) (layer "F.Cu") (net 2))
 (segment (start 142 110) (end 142.05 110.05) (width 0.25) (layer "F.Cu") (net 2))
 (segment (start 148 110) (end 144.55 110) (width 0.25) (layer "F.Cu") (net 2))
 (segment (start 140 110) (end 142 110) (width 0.25) (layer "F.Cu") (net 2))
 (segment (start 135.65 100.95) (end 134.45 100.95) (width 0.25) (layer "F.Cu") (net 2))
 (via (at 134 100.5) (size 0.8) (drill 0.4) (layers "F.Cu" "B.Cu") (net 2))
 (via (at 140 110) (size 0.8) (drill 0.4) (layers "F.Cu" "B.Cu") (free) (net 2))
 (segment (start 134 108.5) (end 134 100.5) (width 0.25) (layer "B.Cu") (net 2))
 (segment (start 140 110) (end 135.5 110) (width 0.25) (layer "B.Cu") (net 2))
 (segment (start 135.5 110) (end 134 108.5) (width 0.25) (layer "B.Cu") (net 2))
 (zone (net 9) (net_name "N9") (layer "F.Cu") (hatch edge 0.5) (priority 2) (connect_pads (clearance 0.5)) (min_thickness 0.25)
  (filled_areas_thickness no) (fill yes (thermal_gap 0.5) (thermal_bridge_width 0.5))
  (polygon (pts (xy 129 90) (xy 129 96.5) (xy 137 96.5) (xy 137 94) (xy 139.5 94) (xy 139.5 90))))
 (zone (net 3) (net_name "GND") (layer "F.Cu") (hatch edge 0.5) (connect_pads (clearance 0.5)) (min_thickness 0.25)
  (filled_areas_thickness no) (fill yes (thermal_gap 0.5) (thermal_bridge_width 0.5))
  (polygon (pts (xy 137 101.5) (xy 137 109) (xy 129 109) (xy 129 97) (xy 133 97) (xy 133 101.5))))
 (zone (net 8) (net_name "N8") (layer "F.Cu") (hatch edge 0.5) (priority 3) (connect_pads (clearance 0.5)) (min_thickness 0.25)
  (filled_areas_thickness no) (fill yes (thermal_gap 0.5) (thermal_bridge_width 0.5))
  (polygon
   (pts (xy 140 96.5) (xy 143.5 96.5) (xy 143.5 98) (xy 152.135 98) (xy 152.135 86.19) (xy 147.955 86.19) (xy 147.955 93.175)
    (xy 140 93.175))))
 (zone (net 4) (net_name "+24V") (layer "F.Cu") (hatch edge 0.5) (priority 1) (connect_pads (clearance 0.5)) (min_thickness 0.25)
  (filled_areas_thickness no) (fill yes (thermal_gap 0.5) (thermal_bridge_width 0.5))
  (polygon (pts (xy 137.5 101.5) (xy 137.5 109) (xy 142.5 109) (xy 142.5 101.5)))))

